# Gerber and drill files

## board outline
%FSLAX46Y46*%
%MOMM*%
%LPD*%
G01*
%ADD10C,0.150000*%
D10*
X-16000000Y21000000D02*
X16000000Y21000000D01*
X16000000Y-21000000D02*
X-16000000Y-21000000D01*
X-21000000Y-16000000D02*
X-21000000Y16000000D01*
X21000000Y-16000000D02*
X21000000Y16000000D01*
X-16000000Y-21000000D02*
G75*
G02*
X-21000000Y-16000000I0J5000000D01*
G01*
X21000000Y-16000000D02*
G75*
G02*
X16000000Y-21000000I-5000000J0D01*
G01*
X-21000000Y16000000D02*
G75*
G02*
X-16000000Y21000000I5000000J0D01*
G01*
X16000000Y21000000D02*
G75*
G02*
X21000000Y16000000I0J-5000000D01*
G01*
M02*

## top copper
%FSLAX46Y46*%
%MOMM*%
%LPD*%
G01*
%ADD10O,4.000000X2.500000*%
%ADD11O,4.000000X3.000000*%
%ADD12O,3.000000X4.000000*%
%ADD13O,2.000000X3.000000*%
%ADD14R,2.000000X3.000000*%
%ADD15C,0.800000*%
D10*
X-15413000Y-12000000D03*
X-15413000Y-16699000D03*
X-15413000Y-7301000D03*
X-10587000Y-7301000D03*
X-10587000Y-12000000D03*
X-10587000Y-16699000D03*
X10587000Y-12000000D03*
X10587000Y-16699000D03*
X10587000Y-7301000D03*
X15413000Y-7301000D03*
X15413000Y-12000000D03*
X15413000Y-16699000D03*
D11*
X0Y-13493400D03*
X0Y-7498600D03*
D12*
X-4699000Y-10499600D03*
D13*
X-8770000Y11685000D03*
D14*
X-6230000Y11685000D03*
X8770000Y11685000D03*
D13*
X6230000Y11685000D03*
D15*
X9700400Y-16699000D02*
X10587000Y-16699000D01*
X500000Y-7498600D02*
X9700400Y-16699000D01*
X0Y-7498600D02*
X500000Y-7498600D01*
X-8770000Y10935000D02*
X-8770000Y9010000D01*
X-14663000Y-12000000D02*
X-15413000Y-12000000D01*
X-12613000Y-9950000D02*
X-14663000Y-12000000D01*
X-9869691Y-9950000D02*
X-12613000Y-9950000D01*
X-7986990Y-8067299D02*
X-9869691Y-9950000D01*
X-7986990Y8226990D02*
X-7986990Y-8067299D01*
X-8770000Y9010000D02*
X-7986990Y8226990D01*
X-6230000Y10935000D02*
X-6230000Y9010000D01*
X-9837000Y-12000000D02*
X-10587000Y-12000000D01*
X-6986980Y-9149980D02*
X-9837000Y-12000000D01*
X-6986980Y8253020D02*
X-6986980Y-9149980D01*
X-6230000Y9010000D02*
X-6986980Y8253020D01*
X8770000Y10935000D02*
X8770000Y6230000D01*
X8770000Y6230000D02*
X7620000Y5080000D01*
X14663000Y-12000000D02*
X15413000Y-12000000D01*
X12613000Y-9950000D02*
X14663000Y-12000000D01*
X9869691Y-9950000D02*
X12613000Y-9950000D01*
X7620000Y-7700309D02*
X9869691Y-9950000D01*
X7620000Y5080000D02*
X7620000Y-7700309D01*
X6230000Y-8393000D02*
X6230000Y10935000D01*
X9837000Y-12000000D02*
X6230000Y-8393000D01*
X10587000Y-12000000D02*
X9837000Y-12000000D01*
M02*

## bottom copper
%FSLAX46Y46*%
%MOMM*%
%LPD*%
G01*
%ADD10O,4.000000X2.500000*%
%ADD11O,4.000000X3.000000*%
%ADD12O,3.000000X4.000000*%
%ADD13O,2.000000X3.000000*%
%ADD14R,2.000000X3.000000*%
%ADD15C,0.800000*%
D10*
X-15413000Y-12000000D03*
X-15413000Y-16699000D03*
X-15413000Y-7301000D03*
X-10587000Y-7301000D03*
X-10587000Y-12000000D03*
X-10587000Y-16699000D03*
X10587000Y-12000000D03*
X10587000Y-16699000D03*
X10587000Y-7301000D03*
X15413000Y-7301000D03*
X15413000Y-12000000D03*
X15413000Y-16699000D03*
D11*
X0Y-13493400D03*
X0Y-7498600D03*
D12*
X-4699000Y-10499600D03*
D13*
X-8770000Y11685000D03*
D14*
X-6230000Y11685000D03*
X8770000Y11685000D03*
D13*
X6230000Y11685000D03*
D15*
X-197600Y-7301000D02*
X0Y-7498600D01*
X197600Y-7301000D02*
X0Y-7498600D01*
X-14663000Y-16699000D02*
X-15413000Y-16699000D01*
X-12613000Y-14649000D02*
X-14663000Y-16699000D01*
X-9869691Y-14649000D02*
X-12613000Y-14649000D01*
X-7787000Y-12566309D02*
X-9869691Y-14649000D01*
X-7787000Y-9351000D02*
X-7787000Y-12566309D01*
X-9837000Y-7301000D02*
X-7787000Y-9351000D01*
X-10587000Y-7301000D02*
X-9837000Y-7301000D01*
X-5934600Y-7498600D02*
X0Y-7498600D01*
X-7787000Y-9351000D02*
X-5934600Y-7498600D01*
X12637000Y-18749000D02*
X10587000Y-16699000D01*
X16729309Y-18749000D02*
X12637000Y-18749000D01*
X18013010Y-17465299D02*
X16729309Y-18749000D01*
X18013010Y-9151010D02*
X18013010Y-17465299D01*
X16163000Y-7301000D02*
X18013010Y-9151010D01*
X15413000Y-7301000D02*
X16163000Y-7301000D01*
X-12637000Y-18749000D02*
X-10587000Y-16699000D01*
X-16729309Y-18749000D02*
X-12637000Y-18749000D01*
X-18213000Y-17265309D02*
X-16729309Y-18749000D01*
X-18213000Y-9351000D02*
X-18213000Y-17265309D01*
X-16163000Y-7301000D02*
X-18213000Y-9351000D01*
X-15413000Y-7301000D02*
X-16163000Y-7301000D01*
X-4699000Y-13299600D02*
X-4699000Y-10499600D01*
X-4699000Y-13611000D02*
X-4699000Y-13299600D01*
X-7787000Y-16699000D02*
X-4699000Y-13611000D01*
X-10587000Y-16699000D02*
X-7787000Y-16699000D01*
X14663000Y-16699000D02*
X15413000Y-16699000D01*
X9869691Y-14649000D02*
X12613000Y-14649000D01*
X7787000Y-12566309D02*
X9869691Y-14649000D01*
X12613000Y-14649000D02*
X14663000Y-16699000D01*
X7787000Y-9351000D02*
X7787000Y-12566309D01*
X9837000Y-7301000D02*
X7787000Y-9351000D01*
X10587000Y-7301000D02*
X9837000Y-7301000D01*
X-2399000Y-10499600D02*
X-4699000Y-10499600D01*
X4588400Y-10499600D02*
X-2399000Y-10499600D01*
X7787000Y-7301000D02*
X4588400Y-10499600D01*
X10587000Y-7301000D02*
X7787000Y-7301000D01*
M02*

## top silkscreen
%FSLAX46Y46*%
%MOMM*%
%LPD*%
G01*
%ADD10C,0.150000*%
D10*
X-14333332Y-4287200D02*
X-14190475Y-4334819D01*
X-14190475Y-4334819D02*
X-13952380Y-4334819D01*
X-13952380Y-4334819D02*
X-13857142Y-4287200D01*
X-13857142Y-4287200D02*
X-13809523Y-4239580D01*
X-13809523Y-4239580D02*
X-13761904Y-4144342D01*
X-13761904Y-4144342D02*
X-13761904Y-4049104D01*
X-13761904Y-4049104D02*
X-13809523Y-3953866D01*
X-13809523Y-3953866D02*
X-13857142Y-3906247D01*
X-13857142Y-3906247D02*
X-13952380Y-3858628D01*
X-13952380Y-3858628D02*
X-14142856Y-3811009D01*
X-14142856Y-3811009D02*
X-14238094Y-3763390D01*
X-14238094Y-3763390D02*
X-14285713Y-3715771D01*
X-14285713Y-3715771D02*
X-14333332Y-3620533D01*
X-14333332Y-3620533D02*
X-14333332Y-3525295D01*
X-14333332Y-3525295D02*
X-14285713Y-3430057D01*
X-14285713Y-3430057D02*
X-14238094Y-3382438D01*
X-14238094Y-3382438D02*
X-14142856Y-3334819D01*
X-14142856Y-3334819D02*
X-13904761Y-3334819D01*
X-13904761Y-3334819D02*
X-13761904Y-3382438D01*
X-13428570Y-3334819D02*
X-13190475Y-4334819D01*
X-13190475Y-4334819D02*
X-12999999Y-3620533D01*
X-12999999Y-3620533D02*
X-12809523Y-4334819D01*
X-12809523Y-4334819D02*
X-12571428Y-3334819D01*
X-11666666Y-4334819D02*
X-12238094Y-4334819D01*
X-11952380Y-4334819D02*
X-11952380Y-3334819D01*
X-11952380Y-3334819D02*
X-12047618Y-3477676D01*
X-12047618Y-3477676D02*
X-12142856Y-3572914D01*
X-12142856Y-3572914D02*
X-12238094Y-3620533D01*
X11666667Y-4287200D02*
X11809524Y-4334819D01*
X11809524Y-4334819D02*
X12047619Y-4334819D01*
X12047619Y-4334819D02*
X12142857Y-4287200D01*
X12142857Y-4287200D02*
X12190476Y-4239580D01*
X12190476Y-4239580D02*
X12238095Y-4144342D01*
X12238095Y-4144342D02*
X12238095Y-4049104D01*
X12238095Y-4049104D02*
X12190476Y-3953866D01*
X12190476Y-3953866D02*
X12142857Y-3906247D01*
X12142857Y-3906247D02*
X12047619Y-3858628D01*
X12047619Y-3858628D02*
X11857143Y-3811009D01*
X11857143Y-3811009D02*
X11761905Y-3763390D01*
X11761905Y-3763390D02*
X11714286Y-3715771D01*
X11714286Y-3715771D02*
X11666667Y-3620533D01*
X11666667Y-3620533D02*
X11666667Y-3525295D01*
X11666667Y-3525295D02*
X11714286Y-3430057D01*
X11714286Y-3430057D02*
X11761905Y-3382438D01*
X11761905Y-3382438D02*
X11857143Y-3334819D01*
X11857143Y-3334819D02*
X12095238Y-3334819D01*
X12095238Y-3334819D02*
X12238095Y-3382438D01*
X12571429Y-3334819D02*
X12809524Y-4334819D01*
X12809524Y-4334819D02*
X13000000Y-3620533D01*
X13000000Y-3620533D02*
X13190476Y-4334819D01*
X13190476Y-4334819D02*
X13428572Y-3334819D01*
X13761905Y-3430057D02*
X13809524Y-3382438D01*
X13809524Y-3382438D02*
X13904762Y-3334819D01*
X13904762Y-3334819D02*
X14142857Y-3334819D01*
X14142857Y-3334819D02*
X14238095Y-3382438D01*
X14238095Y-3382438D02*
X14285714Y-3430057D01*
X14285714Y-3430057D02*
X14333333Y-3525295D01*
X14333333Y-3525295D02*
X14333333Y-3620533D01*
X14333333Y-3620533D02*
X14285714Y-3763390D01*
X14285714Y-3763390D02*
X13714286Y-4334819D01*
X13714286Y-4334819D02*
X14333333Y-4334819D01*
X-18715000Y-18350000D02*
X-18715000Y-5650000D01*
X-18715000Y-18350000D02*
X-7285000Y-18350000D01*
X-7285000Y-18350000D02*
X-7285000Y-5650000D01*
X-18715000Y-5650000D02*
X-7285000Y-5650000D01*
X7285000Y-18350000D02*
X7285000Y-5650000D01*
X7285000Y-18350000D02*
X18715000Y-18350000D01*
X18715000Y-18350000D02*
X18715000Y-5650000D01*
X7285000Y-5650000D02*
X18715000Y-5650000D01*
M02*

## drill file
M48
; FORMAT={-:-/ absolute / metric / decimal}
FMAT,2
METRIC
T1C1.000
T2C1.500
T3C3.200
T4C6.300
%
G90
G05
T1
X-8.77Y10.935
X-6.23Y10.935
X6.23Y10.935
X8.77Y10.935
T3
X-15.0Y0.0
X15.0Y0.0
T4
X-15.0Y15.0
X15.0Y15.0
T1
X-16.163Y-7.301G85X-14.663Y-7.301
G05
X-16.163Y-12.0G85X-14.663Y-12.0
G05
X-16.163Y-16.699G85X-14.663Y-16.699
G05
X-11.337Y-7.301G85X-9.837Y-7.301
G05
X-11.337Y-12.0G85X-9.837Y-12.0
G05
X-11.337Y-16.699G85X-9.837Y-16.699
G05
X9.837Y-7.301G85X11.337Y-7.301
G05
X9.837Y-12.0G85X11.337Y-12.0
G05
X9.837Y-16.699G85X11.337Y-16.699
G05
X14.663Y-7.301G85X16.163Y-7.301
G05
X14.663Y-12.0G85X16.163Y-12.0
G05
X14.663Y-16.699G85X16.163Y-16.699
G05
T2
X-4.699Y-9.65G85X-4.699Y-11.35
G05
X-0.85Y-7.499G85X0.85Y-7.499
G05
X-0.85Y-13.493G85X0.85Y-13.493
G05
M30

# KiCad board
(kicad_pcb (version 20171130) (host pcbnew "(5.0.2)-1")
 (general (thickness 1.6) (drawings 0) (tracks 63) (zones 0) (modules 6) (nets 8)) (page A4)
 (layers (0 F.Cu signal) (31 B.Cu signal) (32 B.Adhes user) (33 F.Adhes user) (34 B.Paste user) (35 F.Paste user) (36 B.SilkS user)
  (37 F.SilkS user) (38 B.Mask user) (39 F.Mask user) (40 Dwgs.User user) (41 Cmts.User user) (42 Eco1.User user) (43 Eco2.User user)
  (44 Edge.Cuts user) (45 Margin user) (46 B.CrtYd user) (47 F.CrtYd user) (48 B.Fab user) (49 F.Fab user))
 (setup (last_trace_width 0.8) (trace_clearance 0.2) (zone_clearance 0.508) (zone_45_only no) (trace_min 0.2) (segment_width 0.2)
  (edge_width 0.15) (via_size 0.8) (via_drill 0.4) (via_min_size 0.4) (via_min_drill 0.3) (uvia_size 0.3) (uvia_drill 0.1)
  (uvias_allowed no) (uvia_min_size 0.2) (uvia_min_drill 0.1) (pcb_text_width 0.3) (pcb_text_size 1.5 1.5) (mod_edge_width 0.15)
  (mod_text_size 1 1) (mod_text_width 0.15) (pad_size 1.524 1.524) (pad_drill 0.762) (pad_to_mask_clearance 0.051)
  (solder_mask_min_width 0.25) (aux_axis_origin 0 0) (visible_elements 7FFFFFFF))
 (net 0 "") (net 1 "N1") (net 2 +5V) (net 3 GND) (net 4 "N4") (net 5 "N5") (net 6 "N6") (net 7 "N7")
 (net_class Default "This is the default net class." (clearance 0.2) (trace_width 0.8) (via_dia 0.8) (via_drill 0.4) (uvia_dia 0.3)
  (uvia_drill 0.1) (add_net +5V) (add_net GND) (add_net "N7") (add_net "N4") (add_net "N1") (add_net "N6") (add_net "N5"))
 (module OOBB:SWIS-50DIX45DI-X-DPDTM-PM (layer F.Cu) (at -15.413 7.301)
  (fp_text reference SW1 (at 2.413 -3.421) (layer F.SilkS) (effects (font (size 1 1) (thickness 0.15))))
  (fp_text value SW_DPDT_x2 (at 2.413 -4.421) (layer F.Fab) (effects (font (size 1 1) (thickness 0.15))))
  (fp_line (start -3.302 11.049) (end -3.302 -1.651) (layer F.SilkS) (width 0.15))
  (fp_line (start -3.302 11.049) (end 8.128 11.049) (layer F.SilkS) (width 0.15))
  (fp_line (start 8.128 11.049) (end 8.128 -1.651) (layer F.SilkS) (width 0.15))
  (fp_line (start -3.302 -1.651) (end 8.128 -1.651) (layer F.SilkS) (width 0.15))
  (pad 2 thru_hole oval (at 0 4.699) (size 4 2.5) (drill oval 2.5 1) (layers *.Cu *.Mask) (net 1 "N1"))
  (pad 1 thru_hole oval (at 0 9.398) (size 4 2.5) (drill oval 2.5 1) (layers *.Cu *.Mask) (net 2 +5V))
  (pad 3 thru_hole oval (at 0 0) (size 4 2.5) (drill oval 2.5 1) (layers *.Cu *.Mask) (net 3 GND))
  (pad 6 thru_hole oval (at 4.826 0) (size 4 2.5) (drill oval 2.5 1) (layers *.Cu *.Mask Eco1.User Eco2.User) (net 2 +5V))
  (pad 5 thru_hole oval (at 4.826 4.699) (size 4 2.5) (drill oval 2.5 1) (layers *.Cu *.Mask) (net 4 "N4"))
  (pad 4 thru_hole oval (at 4.826 9.398) (size 4 2.5) (drill oval 2.5 1) (layers *.Cu *.Mask) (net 3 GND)))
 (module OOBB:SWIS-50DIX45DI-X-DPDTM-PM (layer F.Cu) (at 10.587 7.301)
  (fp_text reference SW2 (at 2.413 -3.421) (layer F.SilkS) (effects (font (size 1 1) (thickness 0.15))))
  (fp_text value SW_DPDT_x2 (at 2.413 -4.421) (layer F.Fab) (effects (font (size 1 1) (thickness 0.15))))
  (fp_line (start -3.302 11.049) (end -3.302 -1.651) (layer F.SilkS) (width 0.15))
  (fp_line (start -3.302 11.049) (end 8.128 11.049) (layer F.SilkS) (width 0.15))
  (fp_line (start 8.128 11.049) (end 8.128 -1.651) (layer F.SilkS) (width 0.15))
  (fp_line (start -3.302 -1.651) (end 8.128 -1.651) (layer F.SilkS) (width 0.15))
  (pad 2 thru_hole oval (at 0 4.699) (size 4 2.5) (drill oval 2.5 1) (layers *.Cu *.Mask) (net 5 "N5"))
  (pad 1 thru_hole oval (at 0 9.398) (size 4 2.5) (drill oval 2.5 1) (layers *.Cu *.Mask) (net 2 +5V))
  (pad 3 thru_hole oval (at 0 0) (size 4 2.5) (drill oval 2.5 1) (layers *.Cu *.Mask) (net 3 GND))
  (pad 6 thru_hole oval (at 4.826 0) (size 4 2.5) (drill oval 2.5 1) (layers *.Cu *.Mask Eco1.User Eco2.User) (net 2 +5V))
  (pad 5 thru_hole oval (at 4.826 4.699) (size 4 2.5) (drill oval 2.5 1) (layers *.Cu *.Mask) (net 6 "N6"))
  (pad 4 thru_hole oval (at 4.826 9.398) (size 4 2.5) (drill oval 2.5 1) (layers *.Cu *.Mask) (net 3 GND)))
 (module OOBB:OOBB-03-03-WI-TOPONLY (layer F.Cu) (at 0 0)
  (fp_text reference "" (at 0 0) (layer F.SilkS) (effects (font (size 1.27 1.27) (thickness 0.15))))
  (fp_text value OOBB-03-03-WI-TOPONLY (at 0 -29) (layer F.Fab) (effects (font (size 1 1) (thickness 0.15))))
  (fp_line (start -16 -21) (end 16 -21) (layer Edge.Cuts) (width 0.15))
  (fp_line (start 16 21) (end -16 21) (layer Edge.Cuts) (width 0.15))
  (fp_line (start -21 16) (end -21 -16) (layer Edge.Cuts) (width 0.15))
  (fp_line (start 21 16) (end 21 -16) (layer Edge.Cuts) (width 0.15))
  (fp_arc (start -16 16) (end -16 21) (angle 90) (layer Edge.Cuts) (width 0.15))
  (fp_arc (start 16 16) (end 16 21) (angle -90) (layer Edge.Cuts) (width 0.15))
  (fp_arc (start -16 -16) (end -16 -21) (angle -90) (layer Edge.Cuts) (width 0.15))
  (fp_arc (start 16 -16) (end 16 -21) (angle 90) (layer Edge.Cuts) (width 0.15))
  (pad "" np_thru_hole circle (at 15 0) (size 3.2 3.2) (drill 3.2) (layers *.Cu *.Mask))
  (pad "" np_thru_hole circle (at 15 -15) (size 6.3 6.3) (drill 6.3) (layers *.Cu *.Mask))
  (pad "" np_thru_hole circle (at -15 0) (size 3.2 3.2) (drill 3.2) (layers *.Cu *.Mask))
  (pad "" np_thru_hole circle (at -15 -15) (size 6.3 6.3) (drill 6.3) (layers *.Cu *.Mask)))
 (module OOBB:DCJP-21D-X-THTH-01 (layer B.Cu) (at 0 13.7 90)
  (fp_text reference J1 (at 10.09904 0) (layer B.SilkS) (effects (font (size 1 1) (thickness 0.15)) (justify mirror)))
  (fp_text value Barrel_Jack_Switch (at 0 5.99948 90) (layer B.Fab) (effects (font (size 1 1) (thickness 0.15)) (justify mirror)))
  (pad 2 thru_hole oval (at 0.2066 0 90) (size 3 4) (drill oval 1.5 3.2) (layers *.Cu *.Mask) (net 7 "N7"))
  (pad 1 thru_hole oval (at 6.2014 0 90) (size 3 4) (drill oval 1.5 3.2) (layers *.Cu *.Mask) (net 2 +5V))
  (pad 3 thru_hole oval (at 3.2004 -4.699) (size 3 4) (drill oval 1.5 3.2) (layers *.Cu *.Mask) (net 3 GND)))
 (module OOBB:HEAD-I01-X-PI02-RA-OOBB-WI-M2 (layer B.Cu) (at -6.23 -10.935 90)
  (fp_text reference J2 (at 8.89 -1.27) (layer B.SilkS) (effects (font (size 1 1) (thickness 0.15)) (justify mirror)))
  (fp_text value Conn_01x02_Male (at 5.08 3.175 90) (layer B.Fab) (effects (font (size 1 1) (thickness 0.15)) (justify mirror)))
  (pad 2 thru_hole oval (at 0 -2.54 90) (size 3 2) (drill 1 (offset 0.75 0)) (layers *.Cu *.Mask) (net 1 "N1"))
  (pad 1 thru_hole rect (at 0 0 90) (size 3 2) (drill 1 (offset 0.75 0)) (layers *.Cu *.Mask) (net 4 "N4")))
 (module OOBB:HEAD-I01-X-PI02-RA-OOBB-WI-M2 (layer B.Cu) (at 8.77 -10.935 90)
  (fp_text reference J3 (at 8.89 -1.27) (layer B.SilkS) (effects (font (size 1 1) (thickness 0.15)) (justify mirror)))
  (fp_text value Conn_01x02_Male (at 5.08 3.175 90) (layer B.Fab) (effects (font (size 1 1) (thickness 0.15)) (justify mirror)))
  (pad 1 thru_hole rect (at 0 0 90) (size 3 2) (drill 1 (offset 0.75 0)) (layers *.Cu *.Mask) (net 6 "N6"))
  (pad 2 thru_hole oval (at 0 -2.54 90) (size 3 2) (drill 1 (offset 0.75 0)) (layers *.Cu *.Mask) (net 5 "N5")))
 (segment (start -0.1976 7.301) (end 0 7.4986) (width 0.8) (layer B.Cu) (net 2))
 (segment (start 0.1976 7.301) (end 0 7.4986) (width 0.8) (layer B.Cu) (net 2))
 (segment (start -14.663 16.699) (end -15.413 16.699) (width 0.8) (layer B.Cu) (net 2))
 (segment (start -12.613 14.649) (end -14.663 16.699) (width 0.8) (layer B.Cu) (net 2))
 (segment (start -9.869691 14.649) (end -12.613 14.649) (width 0.8) (layer B.Cu) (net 2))
 (segment (start -7.787 12.566309) (end -9.869691 14.649) (width 0.8) (layer B.Cu) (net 2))
 (segment (start -7.787 9.351) (end -7.787 12.566309) (width 0.8) (layer B.Cu) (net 2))
 (segment (start -9.837 7.301) (end -7.787 9.351) (width 0.8) (layer B.Cu) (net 2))
 (segment (start -10.587 7.301) (end -9.837 7.301) (width 0.8) (layer B.Cu) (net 2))
 (segment (start -5.9346 7.4986) (end 0 7.4986) (width 0.8) (layer B.Cu) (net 2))
 (segment (start -7.787 9.351) (end -5.9346 7.4986) (width 0.8) (layer B.Cu) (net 2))
 (segment (start 12.637 18.749) (end 10.587 16.699) (width 0.8) (layer B.Cu) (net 2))
 (segment (start 16.729309 18.749) (end 12.637 18.749) (width 0.8) (layer B.Cu) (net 2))
 (segment (start 18.01301 17.465299) (end 16.729309 18.749) (width 0.8) (layer B.Cu) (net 2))
 (segment (start 18.01301 9.15101) (end 18.01301 17.465299) (width 0.8) (layer B.Cu) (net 2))
 (segment (start 16.163 7.301) (end 18.01301 9.15101) (width 0.8) (layer B.Cu) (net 2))
 (segment (start 15.413 7.301) (end 16.163 7.301) (width 0.8) (layer B.Cu) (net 2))
 (segment (start 9.7004 16.699) (end 10.587 16.699) (width 0.8) (layer F.Cu) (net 2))
 (segment (start 0.5 7.4986) (end 9.7004 16.699) (width 0.8) (layer F.Cu) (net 2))
 (segment (start 0 7.4986) (end 0.5 7.4986) (width 0.8) (layer F.Cu) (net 2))
 (segment (start -12.637 18.749) (end -10.587 16.699) (width 0.8) (layer B.Cu) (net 3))
 (segment (start -16.729309 18.749) (end -12.637 18.749) (width 0.8) (layer B.Cu) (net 3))
 (segment (start -18.213 17.265309) (end -16.729309 18.749) (width 0.8) (layer B.Cu) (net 3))
 (segment (start -18.213 9.351) (end -18.213 17.265309) (width 0.8) (layer B.Cu) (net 3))
 (segment (start -16.163 7.301) (end -18.213 9.351) (width 0.8) (layer B.Cu) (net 3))
 (segment (start -15.413 7.301) (end -16.163 7.301) (width 0.8) (layer B.Cu) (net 3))
 (segment (start -4.699 13.2996) (end -4.699 10.4996) (width 0.8) (layer B.Cu) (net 3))
 (segment (start -4.699 13.611) (end -4.699 13.2996) (width 0.8) (layer B.Cu) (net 3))
 (segment (start -7.787 16.699) (end -4.699 13.611) (width 0.8) (layer B.Cu) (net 3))
 (segment (start -10.587 16.699) (end -7.787 16.699) (width 0.8) (layer B.Cu) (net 3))
 (segment (start 14.663 16.699) (end 15.413 16.699) (width 0.8) (layer B.Cu) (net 3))
 (segment (start 9.869691 14.649) (end 12.613 14.649) (width 0.8) (layer B.Cu) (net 3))
 (segment (start 7.787 12.566309) (end 9.869691 14.649) (width 0.8) (layer B.Cu) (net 3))
 (segment (start 12.613 14.649) (end 14.663 16.699) (width 0.8) (layer B.Cu) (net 3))
 (segment (start 7.787 9.351) (end 7.787 12.566309) (width 0.8) (layer B.Cu) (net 3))
 (segment (start 9.837 7.301) (end 7.787 9.351) (width 0.8) (layer B.Cu) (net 3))
 (segment (start 10.587 7.301) (end 9.837 7.301) (width 0.8) (layer B.Cu) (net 3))
 (segment (start -2.399 10.4996) (end -4.699 10.4996) (width 0.8) (layer B.Cu) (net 3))
 (segment (start 4.5884 10.4996) (end -2.399 10.4996) (width 0.8) (layer B.Cu) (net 3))
 (segment (start 7.787 7.301) (end 4.5884 10.4996) (width 0.8) (layer B.Cu) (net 3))
 (segment (start 10.587 7.301) (end 7.787 7.301) (width 0.8) (layer B.Cu) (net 3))
 (segment (start -8.77 -10.935) (end -8.77 -9.01) (width 0.8) (layer F.Cu) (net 1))
 (segment (start -14.663 12) (end -15.413 12) (width 0.8) (layer F.Cu) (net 1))
 (segment (start -12.613 9.95) (end -14.663 12) (width 0.8) (layer F.Cu) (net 1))
 (segment (start -9.869691 9.95) (end -12.613 9.95) (width 0.8) (layer F.Cu) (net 1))
 (segment (start -7.98699 8.067299) (end -9.869691 9.95) (width 0.8) (layer F.Cu) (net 1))
 (segment (start -7.98699 -8.22699) (end -7.98699 8.067299) (width 0.8) (layer F.Cu) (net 1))
 (segment (start -8.77 -9.01) (end -7.98699 -8.22699) (width 0.8) (layer F.Cu) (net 1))
 (segment (start -6.23 -10.935) (end -6.23 -9.01) (width 0.8) (layer F.Cu) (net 4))
 (segment (start -9.837 12) (end -10.587 12) (width 0.8) (layer F.Cu) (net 4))
 (segment (start -6.98698 9.14998) (end -9.837 12) (width 0.8) (layer F.Cu) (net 4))
 (segment (start -6.98698 -8.25302) (end -6.98698 9.14998) (width 0.8) (layer F.Cu) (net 4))
 (segment (start -6.23 -9.01) (end -6.98698 -8.25302) (width 0.8) (layer F.Cu) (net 4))
 (segment (start 8.77 -10.935) (end 8.77 -6.23) (width 0.8) (layer F.Cu) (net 6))
 (segment (start 8.77 -6.23) (end 7.62 -5.08) (width 0.8) (layer F.Cu) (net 6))
 (segment (start 14.663 12) (end 15.413 12) (width 0.8) (layer F.Cu) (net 6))
 (segment (start 12.613 9.95) (end 14.663 12) (width 0.8) (layer F.Cu) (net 6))
 (segment (start 9.869691 9.95) (end 12.613 9.95) (width 0.8) (layer F.Cu) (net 6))
 (segment (start 7.62 7.700309) (end 9.869691 9.95) (width 0.8) (layer F.Cu) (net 6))
 (segment (start 7.62 -5.08) (end 7.62 7.700309) (width 0.8) (layer F.Cu) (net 6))
 (segment (start 6.23 8.393) (end 6.23 -10.935) (width 0.8) (layer F.Cu) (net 5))
 (segment (start 9.837 12) (end 6.23 8.393) (width 0.8) (layer F.Cu) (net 5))
 (segment (start 10.587 12) (end 9.837 12) (width 0.8) (layer F.Cu) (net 5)))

